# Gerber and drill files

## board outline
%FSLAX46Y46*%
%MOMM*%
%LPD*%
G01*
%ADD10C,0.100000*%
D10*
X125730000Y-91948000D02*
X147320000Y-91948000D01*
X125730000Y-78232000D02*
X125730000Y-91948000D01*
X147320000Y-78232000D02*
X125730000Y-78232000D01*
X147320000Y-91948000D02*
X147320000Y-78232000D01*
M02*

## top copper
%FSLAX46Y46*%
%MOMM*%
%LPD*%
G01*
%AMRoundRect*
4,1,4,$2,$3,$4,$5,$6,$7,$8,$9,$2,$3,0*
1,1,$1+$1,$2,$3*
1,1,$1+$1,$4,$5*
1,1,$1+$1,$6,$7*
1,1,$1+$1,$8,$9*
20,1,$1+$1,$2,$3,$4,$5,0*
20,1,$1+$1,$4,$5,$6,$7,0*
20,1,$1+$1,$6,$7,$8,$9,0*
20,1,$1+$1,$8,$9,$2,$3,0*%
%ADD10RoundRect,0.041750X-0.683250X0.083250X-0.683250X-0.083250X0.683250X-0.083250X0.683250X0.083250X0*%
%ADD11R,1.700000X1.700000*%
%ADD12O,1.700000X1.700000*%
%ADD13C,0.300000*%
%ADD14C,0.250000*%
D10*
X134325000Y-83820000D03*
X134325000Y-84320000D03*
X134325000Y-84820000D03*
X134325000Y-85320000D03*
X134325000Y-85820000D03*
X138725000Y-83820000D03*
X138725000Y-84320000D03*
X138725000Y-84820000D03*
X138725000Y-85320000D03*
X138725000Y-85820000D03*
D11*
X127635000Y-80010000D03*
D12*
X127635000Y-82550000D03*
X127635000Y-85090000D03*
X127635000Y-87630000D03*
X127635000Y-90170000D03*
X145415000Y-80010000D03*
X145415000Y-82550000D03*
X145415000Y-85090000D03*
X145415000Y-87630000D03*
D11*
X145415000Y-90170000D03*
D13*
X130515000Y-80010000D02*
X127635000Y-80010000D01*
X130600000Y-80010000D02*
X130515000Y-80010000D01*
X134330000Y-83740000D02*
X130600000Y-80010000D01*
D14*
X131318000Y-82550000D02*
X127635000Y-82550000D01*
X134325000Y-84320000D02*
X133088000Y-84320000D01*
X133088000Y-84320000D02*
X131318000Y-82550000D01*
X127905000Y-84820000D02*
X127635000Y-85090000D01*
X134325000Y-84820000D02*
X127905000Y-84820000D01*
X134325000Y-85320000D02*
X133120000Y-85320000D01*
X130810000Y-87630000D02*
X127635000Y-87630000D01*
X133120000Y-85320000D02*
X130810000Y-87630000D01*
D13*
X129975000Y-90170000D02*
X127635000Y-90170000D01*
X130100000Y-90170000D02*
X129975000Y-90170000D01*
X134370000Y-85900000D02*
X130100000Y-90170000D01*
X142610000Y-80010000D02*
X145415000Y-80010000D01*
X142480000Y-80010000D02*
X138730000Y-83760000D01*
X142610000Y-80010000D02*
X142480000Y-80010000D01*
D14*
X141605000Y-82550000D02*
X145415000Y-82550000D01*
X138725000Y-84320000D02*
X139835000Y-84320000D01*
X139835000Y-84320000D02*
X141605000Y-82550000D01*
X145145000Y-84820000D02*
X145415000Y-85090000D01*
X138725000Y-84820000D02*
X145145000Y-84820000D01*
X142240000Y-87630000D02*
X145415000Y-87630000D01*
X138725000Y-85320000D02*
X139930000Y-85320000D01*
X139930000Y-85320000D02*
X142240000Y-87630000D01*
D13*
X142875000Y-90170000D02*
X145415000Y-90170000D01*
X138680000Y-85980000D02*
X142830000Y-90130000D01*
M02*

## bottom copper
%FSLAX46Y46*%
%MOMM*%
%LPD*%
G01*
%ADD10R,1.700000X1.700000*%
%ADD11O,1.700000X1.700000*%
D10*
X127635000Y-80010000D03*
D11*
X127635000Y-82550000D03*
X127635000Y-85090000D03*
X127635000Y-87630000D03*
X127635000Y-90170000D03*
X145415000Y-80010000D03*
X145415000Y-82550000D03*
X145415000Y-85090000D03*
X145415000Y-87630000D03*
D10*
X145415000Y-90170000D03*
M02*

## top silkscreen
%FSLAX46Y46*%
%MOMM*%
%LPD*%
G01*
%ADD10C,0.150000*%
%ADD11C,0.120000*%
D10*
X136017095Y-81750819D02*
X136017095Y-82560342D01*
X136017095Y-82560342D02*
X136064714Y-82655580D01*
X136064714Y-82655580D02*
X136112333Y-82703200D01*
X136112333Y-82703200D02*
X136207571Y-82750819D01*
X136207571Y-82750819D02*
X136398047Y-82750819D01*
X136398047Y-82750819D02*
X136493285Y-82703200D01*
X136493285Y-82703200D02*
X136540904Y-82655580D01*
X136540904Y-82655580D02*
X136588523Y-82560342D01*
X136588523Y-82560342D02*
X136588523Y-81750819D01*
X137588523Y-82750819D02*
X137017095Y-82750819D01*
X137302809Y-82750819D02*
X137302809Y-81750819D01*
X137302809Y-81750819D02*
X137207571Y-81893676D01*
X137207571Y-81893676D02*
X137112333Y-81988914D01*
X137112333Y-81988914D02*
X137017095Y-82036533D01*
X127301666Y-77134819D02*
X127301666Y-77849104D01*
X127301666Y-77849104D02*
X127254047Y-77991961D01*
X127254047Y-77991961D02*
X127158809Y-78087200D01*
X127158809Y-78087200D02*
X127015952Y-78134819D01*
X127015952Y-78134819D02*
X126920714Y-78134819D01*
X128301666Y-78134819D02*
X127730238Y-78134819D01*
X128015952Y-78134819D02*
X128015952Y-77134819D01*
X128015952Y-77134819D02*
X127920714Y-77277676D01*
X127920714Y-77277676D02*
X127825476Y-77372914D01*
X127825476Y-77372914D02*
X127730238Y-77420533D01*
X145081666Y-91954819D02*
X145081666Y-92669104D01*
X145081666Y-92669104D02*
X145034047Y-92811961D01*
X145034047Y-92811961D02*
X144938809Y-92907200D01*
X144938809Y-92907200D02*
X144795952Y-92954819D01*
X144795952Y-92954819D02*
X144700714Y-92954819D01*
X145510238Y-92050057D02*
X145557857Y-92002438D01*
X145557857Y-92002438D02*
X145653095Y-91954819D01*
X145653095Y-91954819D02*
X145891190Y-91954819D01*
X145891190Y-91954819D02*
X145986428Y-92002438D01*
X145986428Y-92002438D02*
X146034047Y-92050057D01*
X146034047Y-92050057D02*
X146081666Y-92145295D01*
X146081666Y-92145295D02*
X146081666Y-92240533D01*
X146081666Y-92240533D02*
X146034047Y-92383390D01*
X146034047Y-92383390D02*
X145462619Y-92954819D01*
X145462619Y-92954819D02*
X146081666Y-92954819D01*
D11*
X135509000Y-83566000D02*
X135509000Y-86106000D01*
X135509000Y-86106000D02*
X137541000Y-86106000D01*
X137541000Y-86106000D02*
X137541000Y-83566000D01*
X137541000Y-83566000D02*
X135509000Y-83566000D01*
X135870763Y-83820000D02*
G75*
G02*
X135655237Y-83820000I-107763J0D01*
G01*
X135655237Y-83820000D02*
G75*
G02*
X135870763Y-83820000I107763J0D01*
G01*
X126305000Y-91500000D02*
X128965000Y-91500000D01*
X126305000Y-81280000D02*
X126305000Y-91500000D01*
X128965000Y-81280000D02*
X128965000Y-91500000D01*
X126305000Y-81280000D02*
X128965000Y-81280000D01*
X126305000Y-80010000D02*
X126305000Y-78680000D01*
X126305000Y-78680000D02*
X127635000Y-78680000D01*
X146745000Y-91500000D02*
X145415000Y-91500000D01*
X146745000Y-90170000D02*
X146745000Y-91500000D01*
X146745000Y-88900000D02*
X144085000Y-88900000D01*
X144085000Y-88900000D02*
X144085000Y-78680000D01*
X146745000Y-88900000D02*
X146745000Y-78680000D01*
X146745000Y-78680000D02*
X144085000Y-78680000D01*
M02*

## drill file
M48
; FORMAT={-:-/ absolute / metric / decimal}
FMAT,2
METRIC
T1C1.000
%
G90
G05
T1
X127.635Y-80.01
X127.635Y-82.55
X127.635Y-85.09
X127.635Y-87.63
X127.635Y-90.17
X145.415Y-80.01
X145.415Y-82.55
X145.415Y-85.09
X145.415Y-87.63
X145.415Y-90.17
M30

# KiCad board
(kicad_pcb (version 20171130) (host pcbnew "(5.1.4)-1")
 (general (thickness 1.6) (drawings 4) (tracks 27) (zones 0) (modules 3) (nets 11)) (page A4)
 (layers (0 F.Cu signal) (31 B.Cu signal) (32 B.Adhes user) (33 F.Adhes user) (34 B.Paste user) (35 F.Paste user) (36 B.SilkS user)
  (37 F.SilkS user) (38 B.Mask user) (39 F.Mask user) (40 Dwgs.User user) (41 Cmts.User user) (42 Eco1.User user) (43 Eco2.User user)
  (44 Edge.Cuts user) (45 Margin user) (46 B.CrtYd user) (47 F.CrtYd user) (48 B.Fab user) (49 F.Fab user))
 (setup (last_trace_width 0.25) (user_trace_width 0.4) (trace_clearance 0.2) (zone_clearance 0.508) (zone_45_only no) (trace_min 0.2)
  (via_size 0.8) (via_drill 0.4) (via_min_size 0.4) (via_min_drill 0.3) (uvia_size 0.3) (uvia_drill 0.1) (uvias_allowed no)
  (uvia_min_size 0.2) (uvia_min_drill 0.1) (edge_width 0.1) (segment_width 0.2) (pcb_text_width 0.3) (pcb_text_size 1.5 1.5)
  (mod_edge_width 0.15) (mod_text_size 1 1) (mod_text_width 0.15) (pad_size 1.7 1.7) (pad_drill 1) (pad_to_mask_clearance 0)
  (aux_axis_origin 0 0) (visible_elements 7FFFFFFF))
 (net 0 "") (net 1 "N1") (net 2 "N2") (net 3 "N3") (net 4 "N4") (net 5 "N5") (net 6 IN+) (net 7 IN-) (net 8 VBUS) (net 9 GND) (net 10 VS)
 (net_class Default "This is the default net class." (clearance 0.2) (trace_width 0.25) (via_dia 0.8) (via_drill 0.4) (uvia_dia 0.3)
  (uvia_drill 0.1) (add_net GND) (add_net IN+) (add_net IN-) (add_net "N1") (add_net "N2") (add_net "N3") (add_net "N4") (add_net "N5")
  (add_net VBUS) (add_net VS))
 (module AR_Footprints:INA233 (layer F.Cu) (at 136.525 83.82)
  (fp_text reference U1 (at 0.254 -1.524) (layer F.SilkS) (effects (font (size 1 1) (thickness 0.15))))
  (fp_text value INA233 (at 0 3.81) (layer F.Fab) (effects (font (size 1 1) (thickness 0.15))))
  (fp_line (start -1.016 -0.254) (end -1.016 2.286) (layer F.SilkS) (width 0.12))
  (fp_line (start -1.016 2.286) (end 1.016 2.286) (layer F.SilkS) (width 0.12))
  (fp_line (start 1.016 2.286) (end 1.016 -0.254) (layer F.SilkS) (width 0.12))
  (fp_line (start 1.016 -0.254) (end -1.016 -0.254) (layer F.SilkS) (width 0.12))
  (fp_circle (center -0.762 0) (end -0.6858 0.0762) (layer F.SilkS) (width 0.12))
  (pad 1 smd roundrect (at -2.2 0 270) (size 0.25 1.45) (layers F.Cu F.Paste F.Mask) (roundrect_rratio 0.167) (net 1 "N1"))
  (pad 2 smd roundrect (at -2.2 0.5 270) (size 0.25 1.45) (layers F.Cu F.Paste F.Mask) (roundrect_rratio 0.167) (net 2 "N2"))
  (pad 3 smd roundrect (at -2.2 1 270) (size 0.25 1.45) (layers F.Cu F.Paste F.Mask) (roundrect_rratio 0.167) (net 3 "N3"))
  (pad 4 smd roundrect (at -2.2 1.5 270) (size 0.25 1.45) (layers F.Cu F.Paste F.Mask) (roundrect_rratio 0.167) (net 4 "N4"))
  (pad 5 smd roundrect (at -2.2 2 270) (size 0.25 1.45) (layers F.Cu F.Paste F.Mask) (roundrect_rratio 0.167) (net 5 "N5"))
  (pad 10 smd roundrect (at 2.2 0 270) (size 0.25 1.45) (layers F.Cu F.Paste F.Mask) (roundrect_rratio 0.167) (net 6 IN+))
  (pad 9 smd roundrect (at 2.2 0.5 270) (size 0.25 1.45) (layers F.Cu F.Paste F.Mask) (roundrect_rratio 0.167) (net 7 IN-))
  (pad 8 smd roundrect (at 2.2 1 270) (size 0.25 1.45) (layers F.Cu F.Paste F.Mask) (roundrect_rratio 0.167) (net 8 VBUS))
  (pad 7 smd roundrect (at 2.2 1.5 270) (size 0.25 1.45) (layers F.Cu F.Paste F.Mask) (roundrect_rratio 0.167) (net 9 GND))
  (pad 6 smd roundrect (at 2.2 2 270) (size 0.25 1.45) (layers F.Cu F.Paste F.Mask) (roundrect_rratio 0.167) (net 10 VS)))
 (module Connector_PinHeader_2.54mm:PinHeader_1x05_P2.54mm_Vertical (layer F.Cu) (at 127.635 80.01)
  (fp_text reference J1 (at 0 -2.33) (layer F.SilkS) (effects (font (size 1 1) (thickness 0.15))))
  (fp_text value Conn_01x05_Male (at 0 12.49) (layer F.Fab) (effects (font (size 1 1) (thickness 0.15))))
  (fp_line (start -1.33 11.49) (end 1.33 11.49) (layer F.SilkS) (width 0.12))
  (fp_line (start -1.33 1.27) (end -1.33 11.49) (layer F.SilkS) (width 0.12))
  (fp_line (start 1.33 1.27) (end 1.33 11.49) (layer F.SilkS) (width 0.12))
  (fp_line (start -1.33 1.27) (end 1.33 1.27) (layer F.SilkS) (width 0.12))
  (fp_line (start -1.33 0) (end -1.33 -1.33) (layer F.SilkS) (width 0.12))
  (fp_line (start -1.33 -1.33) (end 0 -1.33) (layer F.SilkS) (width 0.12))
  (pad 1 thru_hole rect (at 0 0) (size 1.7 1.7) (drill 1) (layers *.Cu *.Mask) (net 1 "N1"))
  (pad 2 thru_hole oval (at 0 2.54) (size 1.7 1.7) (drill 1) (layers *.Cu *.Mask) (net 2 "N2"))
  (pad 3 thru_hole oval (at 0 5.08) (size 1.7 1.7) (drill 1) (layers *.Cu *.Mask) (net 3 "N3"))
  (pad 4 thru_hole oval (at 0 7.62) (size 1.7 1.7) (drill 1) (layers *.Cu *.Mask) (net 4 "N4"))
  (pad 5 thru_hole oval (at 0 10.16) (size 1.7 1.7) (drill 1) (layers *.Cu *.Mask) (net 5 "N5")))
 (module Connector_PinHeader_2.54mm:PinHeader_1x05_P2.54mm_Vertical (layer F.Cu) (at 145.415 90.17 180)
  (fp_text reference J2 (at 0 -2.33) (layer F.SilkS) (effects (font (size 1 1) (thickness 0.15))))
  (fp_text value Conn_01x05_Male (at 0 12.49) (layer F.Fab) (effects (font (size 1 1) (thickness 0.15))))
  (fp_line (start -1.33 -1.33) (end 0 -1.33) (layer F.SilkS) (width 0.12))
  (fp_line (start -1.33 0) (end -1.33 -1.33) (layer F.SilkS) (width 0.12))
  (fp_line (start -1.33 1.27) (end 1.33 1.27) (layer F.SilkS) (width 0.12))
  (fp_line (start 1.33 1.27) (end 1.33 11.49) (layer F.SilkS) (width 0.12))
  (fp_line (start -1.33 1.27) (end -1.33 11.49) (layer F.SilkS) (width 0.12))
  (fp_line (start -1.33 11.49) (end 1.33 11.49) (layer F.SilkS) (width 0.12))
  (pad 5 thru_hole oval (at 0 10.16 180) (size 1.7 1.7) (drill 1) (layers *.Cu *.Mask) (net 6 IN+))
  (pad 4 thru_hole oval (at 0 7.62 180) (size 1.7 1.7) (drill 1) (layers *.Cu *.Mask) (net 7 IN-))
  (pad 3 thru_hole oval (at 0 5.08 180) (size 1.7 1.7) (drill 1) (layers *.Cu *.Mask) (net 8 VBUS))
  (pad 2 thru_hole oval (at 0 2.54 180) (size 1.7 1.7) (drill 1) (layers *.Cu *.Mask) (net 9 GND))
  (pad 1 thru_hole rect (at 0 0 180) (size 1.7 1.7) (drill 1) (layers *.Cu *.Mask) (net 10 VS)))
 (gr_line (start 125.73 91.948) (end 147.32 91.948) (layer Edge.Cuts) (width 0.1))
 (gr_line (start 125.73 78.232) (end 125.73 91.948) (layer Edge.Cuts) (width 0.1))
 (gr_line (start 147.32 78.232) (end 125.73 78.232) (layer Edge.Cuts) (width 0.1))
 (gr_line (start 147.32 91.948) (end 147.32 78.232) (layer Edge.Cuts) (width 0.1))
 (segment (start 130.515 80.01) (end 127.635 80.01) (width 0.3) (layer F.Cu) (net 1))
 (segment (start 130.6 80.01) (end 130.515 80.01) (width 0.3) (layer F.Cu) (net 1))
 (segment (start 134.33 83.74) (end 130.6 80.01) (width 0.3) (layer F.Cu) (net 1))
 (segment (start 131.318 82.55) (end 127.635 82.55) (width 0.25) (layer F.Cu) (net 2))
 (segment (start 134.325 84.32) (end 133.088 84.32) (width 0.25) (layer F.Cu) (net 2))
 (segment (start 133.088 84.32) (end 131.318 82.55) (width 0.25) (layer F.Cu) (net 2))
 (segment (start 127.905 84.82) (end 127.635 85.09) (width 0.25) (layer F.Cu) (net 3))
 (segment (start 134.325 84.82) (end 127.905 84.82) (width 0.25) (layer F.Cu) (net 3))
 (segment (start 134.325 85.32) (end 133.12 85.32) (width 0.25) (layer F.Cu) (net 4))
 (segment (start 130.81 87.63) (end 127.635 87.63) (width 0.25) (layer F.Cu) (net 4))
 (segment (start 133.12 85.32) (end 130.81 87.63) (width 0.25) (layer F.Cu) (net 4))
 (segment (start 129.975 90.17) (end 127.635 90.17) (width 0.3) (layer F.Cu) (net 5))
 (segment (start 130.1 90.17) (end 129.975 90.17) (width 0.3) (layer F.Cu) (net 5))
 (segment (start 134.37 85.9) (end 130.1 90.17) (width 0.3) (layer F.Cu) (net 5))
 (segment (start 142.61 80.01) (end 145.415 80.01) (width 0.3) (layer F.Cu) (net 6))
 (segment (start 142.48 80.01) (end 138.73 83.76) (width 0.3) (layer F.Cu) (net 6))
 (segment (start 142.61 80.01) (end 142.48 80.01) (width 0.3) (layer F.Cu) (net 6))
 (segment (start 141.605 82.55) (end 145.415 82.55) (width 0.25) (layer F.Cu) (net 7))
 (segment (start 138.725 84.32) (end 139.835 84.32) (width 0.25) (layer F.Cu) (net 7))
 (segment (start 139.835 84.32) (end 141.605 82.55) (width 0.25) (layer F.Cu) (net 7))
 (segment (start 145.145 84.82) (end 145.415 85.09) (width 0.25) (layer F.Cu) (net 8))
 (segment (start 138.725 84.82) (end 145.145 84.82) (width 0.25) (layer F.Cu) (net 8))
 (segment (start 142.24 87.63) (end 145.415 87.63) (width 0.25) (layer F.Cu) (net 9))
 (segment (start 138.725 85.32) (end 139.93 85.32) (width 0.25) (layer F.Cu) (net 9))
 (segment (start 139.93 85.32) (end 142.24 87.63) (width 0.25) (layer F.Cu) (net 9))
 (segment (start 142.875 90.17) (end 145.415 90.17) (width 0.3) (layer F.Cu) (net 10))
 (segment (start 138.68 85.98) (end 142.83 90.13) (width 0.3) (layer F.Cu) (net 10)))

